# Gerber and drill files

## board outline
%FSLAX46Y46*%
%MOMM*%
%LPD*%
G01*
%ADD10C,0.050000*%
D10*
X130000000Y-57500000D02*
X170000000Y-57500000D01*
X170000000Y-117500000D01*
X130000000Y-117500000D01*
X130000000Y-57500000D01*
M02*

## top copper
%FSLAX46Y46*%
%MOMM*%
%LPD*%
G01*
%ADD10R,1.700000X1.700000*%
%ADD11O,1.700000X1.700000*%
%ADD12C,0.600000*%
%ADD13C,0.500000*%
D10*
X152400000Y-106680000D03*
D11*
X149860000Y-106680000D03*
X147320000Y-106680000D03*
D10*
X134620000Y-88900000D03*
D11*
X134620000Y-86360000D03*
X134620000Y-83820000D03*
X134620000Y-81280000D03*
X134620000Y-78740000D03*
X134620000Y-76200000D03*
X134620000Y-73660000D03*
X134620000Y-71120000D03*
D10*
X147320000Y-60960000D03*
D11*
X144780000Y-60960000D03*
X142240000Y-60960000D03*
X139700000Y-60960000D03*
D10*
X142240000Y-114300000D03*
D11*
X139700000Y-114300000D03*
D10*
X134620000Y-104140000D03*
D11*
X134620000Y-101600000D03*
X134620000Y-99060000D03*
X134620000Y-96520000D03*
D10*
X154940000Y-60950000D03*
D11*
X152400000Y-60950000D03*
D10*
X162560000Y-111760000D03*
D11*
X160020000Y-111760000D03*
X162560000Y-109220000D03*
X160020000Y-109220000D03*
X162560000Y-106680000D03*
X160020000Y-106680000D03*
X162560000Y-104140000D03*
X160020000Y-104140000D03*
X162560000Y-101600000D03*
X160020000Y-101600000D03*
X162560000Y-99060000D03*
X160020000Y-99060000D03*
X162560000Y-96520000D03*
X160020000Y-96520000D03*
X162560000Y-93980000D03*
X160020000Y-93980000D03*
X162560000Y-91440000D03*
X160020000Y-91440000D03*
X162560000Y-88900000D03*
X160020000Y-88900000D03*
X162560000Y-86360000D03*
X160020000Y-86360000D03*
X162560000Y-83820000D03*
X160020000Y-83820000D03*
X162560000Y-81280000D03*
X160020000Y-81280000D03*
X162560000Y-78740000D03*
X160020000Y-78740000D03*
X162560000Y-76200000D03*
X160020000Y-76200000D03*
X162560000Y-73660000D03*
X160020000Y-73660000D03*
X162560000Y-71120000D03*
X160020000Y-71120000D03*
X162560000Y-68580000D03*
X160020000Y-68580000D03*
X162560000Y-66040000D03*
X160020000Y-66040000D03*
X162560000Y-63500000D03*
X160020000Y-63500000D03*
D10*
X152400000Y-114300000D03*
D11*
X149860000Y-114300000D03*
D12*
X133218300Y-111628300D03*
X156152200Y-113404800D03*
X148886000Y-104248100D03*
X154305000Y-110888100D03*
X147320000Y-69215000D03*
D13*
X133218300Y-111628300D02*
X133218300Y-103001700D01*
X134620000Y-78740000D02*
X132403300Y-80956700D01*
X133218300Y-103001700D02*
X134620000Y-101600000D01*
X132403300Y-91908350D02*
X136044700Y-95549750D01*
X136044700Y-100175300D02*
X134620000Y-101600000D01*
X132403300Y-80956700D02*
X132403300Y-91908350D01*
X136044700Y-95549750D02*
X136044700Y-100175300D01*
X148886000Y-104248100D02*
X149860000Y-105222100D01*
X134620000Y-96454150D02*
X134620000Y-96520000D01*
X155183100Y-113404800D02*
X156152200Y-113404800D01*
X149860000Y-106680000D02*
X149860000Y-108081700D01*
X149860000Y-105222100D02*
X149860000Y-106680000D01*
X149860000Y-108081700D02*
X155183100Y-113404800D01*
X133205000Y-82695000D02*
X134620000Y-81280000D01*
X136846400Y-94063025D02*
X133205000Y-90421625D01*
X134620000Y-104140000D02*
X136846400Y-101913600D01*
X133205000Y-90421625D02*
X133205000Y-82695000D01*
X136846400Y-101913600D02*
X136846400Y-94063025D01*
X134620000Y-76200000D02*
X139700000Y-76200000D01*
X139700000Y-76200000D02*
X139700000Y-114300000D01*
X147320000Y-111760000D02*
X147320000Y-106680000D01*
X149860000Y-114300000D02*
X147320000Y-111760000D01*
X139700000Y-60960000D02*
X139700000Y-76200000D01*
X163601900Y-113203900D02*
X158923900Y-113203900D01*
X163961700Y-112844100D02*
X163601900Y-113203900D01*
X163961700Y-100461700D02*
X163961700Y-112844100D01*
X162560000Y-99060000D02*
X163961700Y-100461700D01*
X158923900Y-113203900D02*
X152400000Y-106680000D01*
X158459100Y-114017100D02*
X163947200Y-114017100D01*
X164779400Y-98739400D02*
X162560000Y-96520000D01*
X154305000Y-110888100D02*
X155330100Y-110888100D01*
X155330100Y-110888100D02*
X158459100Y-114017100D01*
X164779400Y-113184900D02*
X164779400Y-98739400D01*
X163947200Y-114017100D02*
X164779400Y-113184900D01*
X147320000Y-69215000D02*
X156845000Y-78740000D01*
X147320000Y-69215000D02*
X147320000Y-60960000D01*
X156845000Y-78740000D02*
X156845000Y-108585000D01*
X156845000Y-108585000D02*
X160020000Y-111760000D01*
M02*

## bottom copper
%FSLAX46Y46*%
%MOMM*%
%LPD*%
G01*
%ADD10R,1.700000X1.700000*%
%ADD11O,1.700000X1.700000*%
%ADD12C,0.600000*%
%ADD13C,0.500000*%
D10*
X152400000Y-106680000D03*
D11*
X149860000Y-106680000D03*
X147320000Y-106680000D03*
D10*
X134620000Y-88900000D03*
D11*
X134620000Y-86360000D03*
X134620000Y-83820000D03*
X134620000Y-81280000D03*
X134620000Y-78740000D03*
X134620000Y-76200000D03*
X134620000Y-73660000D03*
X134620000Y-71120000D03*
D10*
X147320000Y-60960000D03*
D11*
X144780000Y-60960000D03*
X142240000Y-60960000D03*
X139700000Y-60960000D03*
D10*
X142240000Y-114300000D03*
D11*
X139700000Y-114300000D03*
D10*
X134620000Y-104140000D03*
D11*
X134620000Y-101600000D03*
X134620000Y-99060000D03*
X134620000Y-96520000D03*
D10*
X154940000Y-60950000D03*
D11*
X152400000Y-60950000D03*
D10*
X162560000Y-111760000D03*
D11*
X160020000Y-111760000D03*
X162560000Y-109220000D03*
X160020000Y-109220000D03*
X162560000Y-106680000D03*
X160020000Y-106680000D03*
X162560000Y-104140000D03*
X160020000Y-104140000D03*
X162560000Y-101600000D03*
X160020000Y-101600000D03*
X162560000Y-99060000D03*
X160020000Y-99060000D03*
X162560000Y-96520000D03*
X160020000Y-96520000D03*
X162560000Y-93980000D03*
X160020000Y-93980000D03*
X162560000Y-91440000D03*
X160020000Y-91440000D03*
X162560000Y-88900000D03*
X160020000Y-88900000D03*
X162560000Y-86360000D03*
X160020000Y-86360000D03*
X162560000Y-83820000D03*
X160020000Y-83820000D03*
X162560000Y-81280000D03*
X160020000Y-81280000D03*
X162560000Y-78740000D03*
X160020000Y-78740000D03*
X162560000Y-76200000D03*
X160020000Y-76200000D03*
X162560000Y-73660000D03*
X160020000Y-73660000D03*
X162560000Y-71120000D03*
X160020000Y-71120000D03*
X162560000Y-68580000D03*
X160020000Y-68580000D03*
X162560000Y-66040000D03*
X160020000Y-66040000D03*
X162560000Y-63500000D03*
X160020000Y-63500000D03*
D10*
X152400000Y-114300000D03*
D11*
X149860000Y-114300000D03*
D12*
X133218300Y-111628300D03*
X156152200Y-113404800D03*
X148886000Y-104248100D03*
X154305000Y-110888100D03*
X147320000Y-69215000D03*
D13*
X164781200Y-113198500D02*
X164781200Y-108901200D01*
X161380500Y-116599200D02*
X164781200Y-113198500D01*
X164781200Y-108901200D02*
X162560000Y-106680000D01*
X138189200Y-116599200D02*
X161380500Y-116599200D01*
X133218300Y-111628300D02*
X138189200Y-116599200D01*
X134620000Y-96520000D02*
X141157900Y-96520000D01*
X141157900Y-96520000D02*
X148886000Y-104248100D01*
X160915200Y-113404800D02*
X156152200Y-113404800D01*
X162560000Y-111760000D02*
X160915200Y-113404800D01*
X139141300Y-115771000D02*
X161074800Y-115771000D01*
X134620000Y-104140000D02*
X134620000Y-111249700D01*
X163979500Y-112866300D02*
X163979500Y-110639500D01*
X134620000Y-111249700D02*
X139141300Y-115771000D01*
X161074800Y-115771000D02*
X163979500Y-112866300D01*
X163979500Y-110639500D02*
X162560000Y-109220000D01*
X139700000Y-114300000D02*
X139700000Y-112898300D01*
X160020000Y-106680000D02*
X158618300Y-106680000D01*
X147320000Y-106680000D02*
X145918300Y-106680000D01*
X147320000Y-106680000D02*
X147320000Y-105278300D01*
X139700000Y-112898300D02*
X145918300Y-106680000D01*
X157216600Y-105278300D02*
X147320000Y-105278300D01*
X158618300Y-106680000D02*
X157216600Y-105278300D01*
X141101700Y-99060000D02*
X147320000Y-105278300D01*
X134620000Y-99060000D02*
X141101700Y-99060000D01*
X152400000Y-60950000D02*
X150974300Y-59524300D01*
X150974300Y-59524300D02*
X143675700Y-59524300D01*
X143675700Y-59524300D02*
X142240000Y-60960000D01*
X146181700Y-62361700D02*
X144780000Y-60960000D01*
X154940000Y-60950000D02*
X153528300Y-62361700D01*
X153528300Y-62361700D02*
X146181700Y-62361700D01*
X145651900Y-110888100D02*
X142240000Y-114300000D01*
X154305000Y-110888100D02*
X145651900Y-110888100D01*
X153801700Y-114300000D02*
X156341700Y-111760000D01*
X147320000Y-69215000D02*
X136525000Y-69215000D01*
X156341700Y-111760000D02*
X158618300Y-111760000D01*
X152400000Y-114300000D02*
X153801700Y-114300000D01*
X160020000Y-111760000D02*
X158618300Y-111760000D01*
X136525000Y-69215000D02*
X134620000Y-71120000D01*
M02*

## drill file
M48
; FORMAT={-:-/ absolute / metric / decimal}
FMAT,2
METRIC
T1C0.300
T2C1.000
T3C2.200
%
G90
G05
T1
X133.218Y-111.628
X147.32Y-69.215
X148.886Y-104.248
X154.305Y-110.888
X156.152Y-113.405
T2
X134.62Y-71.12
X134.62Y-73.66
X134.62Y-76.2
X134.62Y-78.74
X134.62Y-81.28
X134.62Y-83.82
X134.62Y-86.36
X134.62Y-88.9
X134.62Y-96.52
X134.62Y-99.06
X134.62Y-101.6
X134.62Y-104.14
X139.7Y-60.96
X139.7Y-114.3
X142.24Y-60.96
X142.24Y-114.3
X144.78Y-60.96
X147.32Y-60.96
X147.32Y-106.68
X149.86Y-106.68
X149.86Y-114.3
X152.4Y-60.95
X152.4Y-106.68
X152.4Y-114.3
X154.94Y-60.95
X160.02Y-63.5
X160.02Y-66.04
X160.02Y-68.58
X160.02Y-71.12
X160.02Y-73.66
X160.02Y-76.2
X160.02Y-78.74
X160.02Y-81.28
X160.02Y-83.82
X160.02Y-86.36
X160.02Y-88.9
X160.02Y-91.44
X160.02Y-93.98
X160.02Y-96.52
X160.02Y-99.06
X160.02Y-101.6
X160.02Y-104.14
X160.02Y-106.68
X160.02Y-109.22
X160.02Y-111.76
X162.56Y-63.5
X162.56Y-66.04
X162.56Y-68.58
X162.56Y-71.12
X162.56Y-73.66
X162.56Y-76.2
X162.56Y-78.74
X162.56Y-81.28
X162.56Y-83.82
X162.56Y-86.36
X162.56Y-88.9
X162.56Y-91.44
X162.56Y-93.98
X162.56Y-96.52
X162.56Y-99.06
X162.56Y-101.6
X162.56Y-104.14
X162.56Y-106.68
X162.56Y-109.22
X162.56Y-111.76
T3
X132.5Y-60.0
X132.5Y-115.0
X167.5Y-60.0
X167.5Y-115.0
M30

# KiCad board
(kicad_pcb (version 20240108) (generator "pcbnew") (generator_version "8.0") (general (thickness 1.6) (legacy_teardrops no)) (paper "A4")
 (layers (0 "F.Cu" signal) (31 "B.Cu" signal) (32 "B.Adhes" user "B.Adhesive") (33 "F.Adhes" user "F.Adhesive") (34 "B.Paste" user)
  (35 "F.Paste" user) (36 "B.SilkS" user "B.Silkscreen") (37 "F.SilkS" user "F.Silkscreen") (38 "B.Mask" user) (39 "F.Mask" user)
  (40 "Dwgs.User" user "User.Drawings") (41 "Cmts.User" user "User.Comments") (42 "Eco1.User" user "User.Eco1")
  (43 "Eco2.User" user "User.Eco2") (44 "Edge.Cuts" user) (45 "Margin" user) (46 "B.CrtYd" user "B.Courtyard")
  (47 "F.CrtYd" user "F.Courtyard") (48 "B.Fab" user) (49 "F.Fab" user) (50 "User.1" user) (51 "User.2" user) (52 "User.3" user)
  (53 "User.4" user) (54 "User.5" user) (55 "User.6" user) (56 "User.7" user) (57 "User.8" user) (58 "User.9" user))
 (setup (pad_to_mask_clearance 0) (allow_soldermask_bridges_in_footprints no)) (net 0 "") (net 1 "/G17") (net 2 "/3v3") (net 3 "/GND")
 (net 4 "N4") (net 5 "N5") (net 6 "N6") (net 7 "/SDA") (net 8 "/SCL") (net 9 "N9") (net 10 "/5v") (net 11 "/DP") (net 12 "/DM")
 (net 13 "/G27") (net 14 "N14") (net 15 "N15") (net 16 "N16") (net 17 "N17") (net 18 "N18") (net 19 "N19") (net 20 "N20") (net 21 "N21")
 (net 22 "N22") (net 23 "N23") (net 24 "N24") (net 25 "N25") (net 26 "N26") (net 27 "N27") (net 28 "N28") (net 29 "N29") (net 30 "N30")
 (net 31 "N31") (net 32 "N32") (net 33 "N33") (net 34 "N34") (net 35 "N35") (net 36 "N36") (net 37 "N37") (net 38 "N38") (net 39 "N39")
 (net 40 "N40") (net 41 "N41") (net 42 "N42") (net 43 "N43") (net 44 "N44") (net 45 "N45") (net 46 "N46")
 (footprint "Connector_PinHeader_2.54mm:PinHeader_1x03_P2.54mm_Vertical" (layer "F.Cu") (at 152.4 106.68 -90)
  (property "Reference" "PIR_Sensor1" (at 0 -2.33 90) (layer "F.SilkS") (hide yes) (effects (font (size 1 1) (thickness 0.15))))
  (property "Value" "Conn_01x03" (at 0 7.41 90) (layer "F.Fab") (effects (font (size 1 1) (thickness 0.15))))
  (pad "1" thru_hole rect (at 0 0 270) (size 1.7 1.7) (drill 1) (layers "*.Cu" "*.Mask") (remove_unused_layers no) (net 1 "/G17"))
  (pad "2" thru_hole oval (at 0 2.54 270) (size 1.7 1.7) (drill 1) (layers "*.Cu" "*.Mask") (remove_unused_layers no) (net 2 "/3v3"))
  (pad "3" thru_hole oval (at 0 5.08 270) (size 1.7 1.7) (drill 1) (layers "*.Cu" "*.Mask") (remove_unused_layers no) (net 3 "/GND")))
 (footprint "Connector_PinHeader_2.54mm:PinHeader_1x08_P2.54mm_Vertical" (layer "F.Cu") (at 134.62 88.9 180)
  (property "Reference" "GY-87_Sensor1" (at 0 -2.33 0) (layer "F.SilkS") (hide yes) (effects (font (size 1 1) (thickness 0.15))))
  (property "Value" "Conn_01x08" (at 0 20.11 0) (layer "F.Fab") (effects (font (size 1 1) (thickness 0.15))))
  (pad "1" thru_hole rect (at 0 0 180) (size 1.7 1.7) (drill 1) (layers "*.Cu" "*.Mask") (remove_unused_layers no) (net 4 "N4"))
  (pad "2" thru_hole oval (at 0 2.54 180) (size 1.7 1.7) (drill 1) (layers "*.Cu" "*.Mask") (remove_unused_layers no) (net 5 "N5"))
  (pad "3" thru_hole oval (at 0 5.08 180) (size 1.7 1.7) (drill 1) (layers "*.Cu" "*.Mask") (remove_unused_layers no) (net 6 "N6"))
  (pad "4" thru_hole oval (at 0 7.62 180) (size 1.7 1.7) (drill 1) (layers "*.Cu" "*.Mask") (remove_unused_layers no) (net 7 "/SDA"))
  (pad "5" thru_hole oval (at 0 10.16 180) (size 1.7 1.7) (drill 1) (layers "*.Cu" "*.Mask") (remove_unused_layers no) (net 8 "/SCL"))
  (pad "6" thru_hole oval (at 0 12.7 180) (size 1.7 1.7) (drill 1) (layers "*.Cu" "*.Mask") (remove_unused_layers no) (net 3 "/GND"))
  (pad "7" thru_hole oval (at 0 15.24 180) (size 1.7 1.7) (drill 1) (layers "*.Cu" "*.Mask") (remove_unused_layers no) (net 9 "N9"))
  (pad "8" thru_hole oval (at 0 17.78 180) (size 1.7 1.7) (drill 1) (layers "*.Cu" "*.Mask") (remove_unused_layers no) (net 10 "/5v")))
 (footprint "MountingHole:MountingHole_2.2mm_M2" (layer "F.Cu") (at 132.5 60)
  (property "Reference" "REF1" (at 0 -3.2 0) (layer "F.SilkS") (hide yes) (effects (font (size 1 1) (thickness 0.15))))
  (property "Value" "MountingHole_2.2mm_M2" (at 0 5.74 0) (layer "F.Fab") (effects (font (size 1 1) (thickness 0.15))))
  (pad "" np_thru_hole circle (at 0 0) (size 2.2 2.2) (drill 2.2) (layers "*.Cu" "*.Mask")))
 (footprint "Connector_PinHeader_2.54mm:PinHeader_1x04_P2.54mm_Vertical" (layer "F.Cu") (at 147.32 60.96 -90)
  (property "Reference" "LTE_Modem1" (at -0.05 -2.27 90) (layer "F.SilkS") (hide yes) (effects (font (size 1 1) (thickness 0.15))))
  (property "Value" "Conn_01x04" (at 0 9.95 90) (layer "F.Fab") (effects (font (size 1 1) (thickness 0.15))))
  (pad "1" thru_hole rect (at 0 0 270) (size 1.7 1.7) (drill 1) (layers "*.Cu" "*.Mask") (remove_unused_layers no) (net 10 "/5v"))
  (pad "2" thru_hole oval (at 0 2.54 270) (size 1.7 1.7) (drill 1) (layers "*.Cu" "*.Mask") (remove_unused_layers no) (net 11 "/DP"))
  (pad "3" thru_hole oval (at 0 5.08 270) (size 1.7 1.7) (drill 1) (layers "*.Cu" "*.Mask") (remove_unused_layers no) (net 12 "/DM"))
  (pad "4" thru_hole oval (at 0 7.62 270) (size 1.7 1.7) (drill 1) (layers "*.Cu" "*.Mask") (remove_unused_layers no) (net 3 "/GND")))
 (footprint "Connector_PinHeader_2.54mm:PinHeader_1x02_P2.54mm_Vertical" (layer "F.Cu") (at 142.24 114.3 -90)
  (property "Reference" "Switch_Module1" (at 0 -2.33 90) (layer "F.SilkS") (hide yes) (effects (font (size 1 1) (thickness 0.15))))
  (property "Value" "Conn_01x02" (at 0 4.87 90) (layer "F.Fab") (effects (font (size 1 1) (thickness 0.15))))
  (pad "1" thru_hole rect (at 0 0 270) (size 1.7 1.7) (drill 1) (layers "*.Cu" "*.Mask") (remove_unused_layers no) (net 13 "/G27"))
  (pad "2" thru_hole oval (at 0 2.54 270) (size 1.7 1.7) (drill 1) (layers "*.Cu" "*.Mask") (remove_unused_layers no) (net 3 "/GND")))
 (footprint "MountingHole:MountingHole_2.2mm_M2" (layer "F.Cu") (at 167.5 115)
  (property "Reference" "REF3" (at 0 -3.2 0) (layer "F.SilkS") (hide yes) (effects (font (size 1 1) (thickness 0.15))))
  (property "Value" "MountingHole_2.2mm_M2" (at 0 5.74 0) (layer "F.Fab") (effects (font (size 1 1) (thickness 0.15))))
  (pad "" np_thru_hole circle (at 0 0) (size 2.2 2.2) (drill 2.2) (layers "*.Cu" "*.Mask")))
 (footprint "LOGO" (layer "F.Cu") (at 144.78 97.79)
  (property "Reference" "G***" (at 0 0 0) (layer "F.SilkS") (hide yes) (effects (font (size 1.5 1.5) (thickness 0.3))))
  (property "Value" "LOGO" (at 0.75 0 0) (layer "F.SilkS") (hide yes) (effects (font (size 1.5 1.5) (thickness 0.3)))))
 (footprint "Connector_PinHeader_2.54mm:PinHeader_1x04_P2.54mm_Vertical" (layer "F.Cu") (at 134.62 104.14 180)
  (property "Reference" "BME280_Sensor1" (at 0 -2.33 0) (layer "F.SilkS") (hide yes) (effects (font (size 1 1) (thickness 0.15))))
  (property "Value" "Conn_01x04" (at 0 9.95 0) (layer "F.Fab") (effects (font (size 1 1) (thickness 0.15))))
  (pad "1" thru_hole rect (at 0 0 180) (size 1.7 1.7) (drill 1) (layers "*.Cu" "*.Mask") (remove_unused_layers no) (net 7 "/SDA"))
  (pad "2" thru_hole oval (at 0 2.54 180) (size 1.7 1.7) (drill 1) (layers "*.Cu" "*.Mask") (remove_unused_layers no) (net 8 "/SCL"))
  (pad "3" thru_hole oval (at 0 5.08 180) (size 1.7 1.7) (drill 1) (layers "*.Cu" "*.Mask") (remove_unused_layers no) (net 3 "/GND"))
  (pad "4" thru_hole oval (at 0 7.62 180) (size 1.7 1.7) (drill 1) (layers "*.Cu" "*.Mask") (remove_unused_layers no) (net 2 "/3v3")))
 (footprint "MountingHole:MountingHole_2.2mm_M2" (layer "F.Cu") (at 132.5 115)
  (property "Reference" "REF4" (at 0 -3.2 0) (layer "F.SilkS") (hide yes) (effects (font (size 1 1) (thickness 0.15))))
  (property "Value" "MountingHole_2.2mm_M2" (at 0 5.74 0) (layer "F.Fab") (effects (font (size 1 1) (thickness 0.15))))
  (pad "" np_thru_hole circle (at 0 0) (size 2.2 2.2) (drill 2.2) (layers "*.Cu" "*.Mask")))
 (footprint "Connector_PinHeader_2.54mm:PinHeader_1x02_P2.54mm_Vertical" (layer "F.Cu") (at 154.94 60.95 -90)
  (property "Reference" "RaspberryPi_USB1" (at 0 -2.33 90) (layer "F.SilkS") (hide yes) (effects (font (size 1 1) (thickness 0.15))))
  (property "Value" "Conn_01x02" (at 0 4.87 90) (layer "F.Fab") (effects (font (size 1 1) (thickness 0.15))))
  (pad "1" thru_hole rect (at 0 0 270) (size 1.7 1.7) (drill 1) (layers "*.Cu" "*.Mask") (remove_unused_layers no) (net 11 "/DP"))
  (pad "2" thru_hole oval (at 0 2.54 270) (size 1.7 1.7) (drill 1) (layers "*.Cu" "*.Mask") (remove_unused_layers no) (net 12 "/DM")))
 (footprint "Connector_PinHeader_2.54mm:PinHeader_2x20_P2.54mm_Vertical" (layer "F.Cu") (at 162.56 111.76 180)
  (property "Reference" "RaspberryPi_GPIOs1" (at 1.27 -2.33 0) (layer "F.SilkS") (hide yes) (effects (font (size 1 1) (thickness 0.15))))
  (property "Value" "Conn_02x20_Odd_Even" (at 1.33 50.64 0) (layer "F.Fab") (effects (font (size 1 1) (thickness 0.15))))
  (pad "1" thru_hole rect (at 0 0 180) (size 1.7 1.7) (drill 1) (layers "*.Cu" "*.Mask") (remove_unused_layers no) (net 2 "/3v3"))
  (pad "2" thru_hole oval (at 2.54 0 180) (size 1.7 1.7) (drill 1) (layers "*.Cu" "*.Mask") (remove_unused_layers no) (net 10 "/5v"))
  (pad "3" thru_hole oval (at 0 2.54 180) (size 1.7 1.7) (drill 1) (layers "*.Cu" "*.Mask") (remove_unused_layers no) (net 7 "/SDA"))
  (pad "4" thru_hole oval (at 2.54 2.54 180) (size 1.7 1.7) (drill 1) (layers "*.Cu" "*.Mask") (remove_unused_layers no) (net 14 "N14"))
  (pad "5" thru_hole oval (at 0 5.08 180) (size 1.7 1.7) (drill 1) (layers "*.Cu" "*.Mask") (remove_unused_layers no) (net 8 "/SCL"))
  (pad "6" thru_hole oval (at 2.54 5.08 180) (size 1.7 1.7) (drill 1) (layers "*.Cu" "*.Mask") (remove_unused_layers no) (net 3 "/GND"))
  (pad "7" thru_hole oval (at 0 7.62 180) (size 1.7 1.7) (drill 1) (layers "*.Cu" "*.Mask") (remove_unused_layers no) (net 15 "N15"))
  (pad "8" thru_hole oval (at 2.54 7.62 180) (size 1.7 1.7) (drill 1) (layers "*.Cu" "*.Mask") (remove_unused_layers no) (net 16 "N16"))
  (pad "9" thru_hole oval (at 0 10.16 180) (size 1.7 1.7) (drill 1) (layers "*.Cu" "*.Mask") (remove_unused_layers no) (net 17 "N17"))
  (pad "10" thru_hole oval (at 2.54 10.16 180) (size 1.7 1.7) (drill 1) (layers "*.Cu" "*.Mask") (remove_unused_layers no) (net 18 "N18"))
  (pad "11" thru_hole oval (at 0 12.7 180) (size 1.7 1.7) (drill 1) (layers "*.Cu" "*.Mask") (remove_unused_layers no) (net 1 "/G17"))
  (pad "12" thru_hole oval (at 2.54 12.7 180) (size 1.7 1.7) (drill 1) (layers "*.Cu" "*.Mask") (remove_unused_layers no) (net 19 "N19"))
  (pad "13" thru_hole oval (at 0 15.24 180) (size 1.7 1.7) (drill 1) (layers "*.Cu" "*.Mask") (remove_unused_layers no) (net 13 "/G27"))
  (pad "14" thru_hole oval (at 2.54 15.24 180) (size 1.7 1.7) (drill 1) (layers "*.Cu" "*.Mask") (remove_unused_layers no) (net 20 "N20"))
  (pad "15" thru_hole oval (at 0 17.78 180) (size 1.7 1.7) (drill 1) (layers "*.Cu" "*.Mask") (remove_unused_layers no) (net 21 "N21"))
  (pad "16" thru_hole oval (at 2.54 17.78 180) (size 1.7 1.7) (drill 1) (layers "*.Cu" "*.Mask") (remove_unused_layers no) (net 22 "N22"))
  (pad "17" thru_hole oval (at 0 20.32 180) (size 1.7 1.7) (drill 1) (layers "*.Cu" "*.Mask") (remove_unused_layers no) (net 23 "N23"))
  (pad "18" thru_hole oval (at 2.54 20.32 180) (size 1.7 1.7) (drill 1) (layers "*.Cu" "*.Mask") (remove_unused_layers no) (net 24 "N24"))
  (pad "19" thru_hole oval (at 0 22.86 180) (size 1.7 1.7) (drill 1) (layers "*.Cu" "*.Mask") (remove_unused_layers no) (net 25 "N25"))
  (pad "20" thru_hole oval (at 2.54 22.86 180) (size 1.7 1.7) (drill 1) (layers "*.Cu" "*.Mask") (remove_unused_layers no) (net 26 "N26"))
  (pad "21" thru_hole oval (at 0 25.4 180) (size 1.7 1.7) (drill 1) (layers "*.Cu" "*.Mask") (remove_unused_layers no) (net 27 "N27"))
  (pad "22" thru_hole oval (at 2.54 25.4 180) (size 1.7 1.7) (drill 1) (layers "*.Cu" "*.Mask") (remove_unused_layers no) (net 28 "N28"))
  (pad "23" thru_hole oval (at 0 27.94 180) (size 1.7 1.7) (drill 1) (layers "*.Cu" "*.Mask") (remove_unused_layers no) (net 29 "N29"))
  (pad "24" thru_hole oval (at 2.54 27.94 180) (size 1.7 1.7) (drill 1) (layers "*.Cu" "*.Mask") (remove_unused_layers no) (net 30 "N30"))
  (pad "25" thru_hole oval (at 0 30.48 180) (size 1.7 1.7) (drill 1) (layers "*.Cu" "*.Mask") (remove_unused_layers no) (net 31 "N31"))
  (pad "26" thru_hole oval (at 2.54 30.48 180) (size 1.7 1.7) (drill 1) (layers "*.Cu" "*.Mask") (remove_unused_layers no) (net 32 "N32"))
  (pad "27" thru_hole oval (at 0 33.02 180) (size 1.7 1.7) (drill 1) (layers "*.Cu" "*.Mask") (remove_unused_layers no) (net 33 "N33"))
  (pad "28" thru_hole oval (at 2.54 33.02 180) (size 1.7 1.7) (drill 1) (layers "*.Cu" "*.Mask") (remove_unused_layers no) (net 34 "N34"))
  (pad "29" thru_hole oval (at 0 35.56 180) (size 1.7 1.7) (drill 1) (layers "*.Cu" "*.Mask") (remove_unused_layers no) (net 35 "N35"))
  (pad "30" thru_hole oval (at 2.54 35.56 180) (size 1.7 1.7) (drill 1) (layers "*.Cu" "*.Mask") (remove_unused_layers no) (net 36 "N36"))
  (pad "31" thru_hole oval (at 0 38.1 180) (size 1.7 1.7) (drill 1) (layers "*.Cu" "*.Mask") (remove_unused_layers no) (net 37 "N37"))
  (pad "32" thru_hole oval (at 2.54 38.1 180) (size 1.7 1.7) (drill 1) (layers "*.Cu" "*.Mask") (remove_unused_layers no) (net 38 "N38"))
  (pad "33" thru_hole oval (at 0 40.64 180) (size 1.7 1.7) (drill 1) (layers "*.Cu" "*.Mask") (remove_unused_layers no) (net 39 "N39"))
  (pad "34" thru_hole oval (at 2.54 40.64 180) (size 1.7 1.7) (drill 1) (layers "*.Cu" "*.Mask") (remove_unused_layers no) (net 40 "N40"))
  (pad "35" thru_hole oval (at 0 43.18 180) (size 1.7 1.7) (drill 1) (layers "*.Cu" "*.Mask") (remove_unused_layers no) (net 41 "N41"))
  (pad "36" thru_hole oval (at 2.54 43.18 180) (size 1.7 1.7) (drill 1) (layers "*.Cu" "*.Mask") (remove_unused_layers no) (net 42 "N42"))
  (pad "37" thru_hole oval (at 0 45.72 180) (size 1.7 1.7) (drill 1) (layers "*.Cu" "*.Mask") (remove_unused_layers no) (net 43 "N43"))
  (pad "38" thru_hole oval (at 2.54 45.72 180) (size 1.7 1.7) (drill 1) (layers "*.Cu" "*.Mask") (remove_unused_layers no) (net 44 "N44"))
  (pad "39" thru_hole oval (at 0 48.26 180) (size 1.7 1.7) (drill 1) (layers "*.Cu" "*.Mask") (remove_unused_layers no) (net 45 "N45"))
  (pad "40" thru_hole oval (at 2.54 48.26 180) (size 1.7 1.7) (drill 1) (layers "*.Cu" "*.Mask") (remove_unused_layers no) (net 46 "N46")))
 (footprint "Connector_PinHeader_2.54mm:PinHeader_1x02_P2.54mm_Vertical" (layer "F.Cu") (at 152.4 114.3 -90)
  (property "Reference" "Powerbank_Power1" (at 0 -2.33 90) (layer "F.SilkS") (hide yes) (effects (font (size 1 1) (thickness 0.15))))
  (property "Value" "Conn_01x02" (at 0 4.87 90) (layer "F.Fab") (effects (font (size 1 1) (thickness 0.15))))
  (pad "1" thru_hole rect (at 0 0 270) (size 1.7 1.7) (drill 1) (layers "*.Cu" "*.Mask") (remove_unused_layers no) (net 10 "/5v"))
  (pad "2" thru_hole oval (at 0 2.54 270) (size 1.7 1.7) (drill 1) (layers "*.Cu" "*.Mask") (remove_unused_layers no) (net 3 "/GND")))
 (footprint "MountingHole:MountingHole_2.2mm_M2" (layer "F.Cu") (at 167.5 60)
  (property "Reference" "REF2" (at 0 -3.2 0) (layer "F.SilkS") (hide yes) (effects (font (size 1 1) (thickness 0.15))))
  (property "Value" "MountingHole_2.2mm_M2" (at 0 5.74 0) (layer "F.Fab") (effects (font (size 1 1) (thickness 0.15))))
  (pad "" np_thru_hole circle (at 0 0) (size 2.2 2.2) (drill 2.2) (layers "*.Cu" "*.Mask")))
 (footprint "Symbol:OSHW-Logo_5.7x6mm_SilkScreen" (layer "F.Cu") (at 152.4 97.79)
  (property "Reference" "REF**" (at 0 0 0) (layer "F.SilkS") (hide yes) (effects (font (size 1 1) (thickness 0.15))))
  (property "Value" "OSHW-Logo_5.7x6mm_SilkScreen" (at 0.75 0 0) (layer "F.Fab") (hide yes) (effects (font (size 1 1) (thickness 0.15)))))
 (gr_rect (start 130 57.5) (end 170 117.5) (stroke (width 0.05) (type default)) (fill none) (layer "Edge.Cuts"))
 (segment (start 133.2183 111.6283) (end 133.2183 103.0017) (width 0.5) (layer "F.Cu") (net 8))
 (segment (start 134.62 78.74) (end 132.4033 80.9567) (width 0.5) (layer "F.Cu") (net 8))
 (segment (start 133.2183 103.0017) (end 134.62 101.6) (width 0.5) (layer "F.Cu") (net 8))
 (segment (start 132.4033 91.90835) (end 136.0447 95.54975) (width 0.5) (layer "F.Cu") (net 8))
 (segment (start 136.0447 100.1753) (end 134.62 101.6) (width 0.5) (layer "F.Cu") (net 8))
 (segment (start 132.4033 80.9567) (end 132.4033 91.90835) (width 0.5) (layer "F.Cu") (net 8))
 (segment (start 136.0447 95.54975) (end 136.0447 100.1753) (width 0.5) (layer "F.Cu") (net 8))
 (via (at 133.2183 111.6283) (size 0.6) (drill 0.3) (layers "F.Cu" "B.Cu") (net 8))
 (segment (start 164.7812 113.1985) (end 164.7812 108.9012) (width 0.5) (layer "B.Cu") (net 8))
 (segment (start 161.3805 116.5992) (end 164.7812 113.1985) (width 0.5) (layer "B.Cu") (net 8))
 (segment (start 164.7812 108.9012) (end 162.56 106.68) (width 0.5) (layer "B.Cu") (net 8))
 (segment (start 138.1892 116.5992) (end 161.3805 116.5992) (width 0.5) (layer "B.Cu") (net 8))
 (segment (start 133.2183 111.6283) (end 138.1892 116.5992) (width 0.5) (layer "B.Cu") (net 8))
 (segment (start 148.886 104.2481) (end 149.86 105.2221) (width 0.5) (layer "F.Cu") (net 2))
 (segment (start 134.62 96.45415) (end 134.62 96.52) (width 0.5) (layer "F.Cu") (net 2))
 (segment (start 155.1831 113.4048) (end 156.1522 113.4048) (width 0.5) (layer "F.Cu") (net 2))
 (segment (start 149.86 106.68) (end 149.86 108.0817) (width 0.5) (layer "F.Cu") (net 2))
 (segment (start 149.86 105.2221) (end 149.86 106.68) (width 0.5) (layer "F.Cu") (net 2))
 (segment (start 149.86 108.0817) (end 155.1831 113.4048) (width 0.5) (layer "F.Cu") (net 2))
 (via (at 156.1522 113.4048) (size 0.6) (drill 0.3) (layers "F.Cu" "B.Cu") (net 2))
 (via (at 148.886 104.2481) (size 0.6) (drill 0.3) (layers "F.Cu" "B.Cu") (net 2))
 (segment (start 134.62 96.52) (end 141.1579 96.52) (width 0.5) (layer "B.Cu") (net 2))
 (segment (start 141.1579 96.52) (end 148.886 104.2481) (width 0.5) (layer "B.Cu") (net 2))
 (segment (start 160.9152 113.4048) (end 156.1522 113.4048) (width 0.5) (layer "B.Cu") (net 2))
 (segment (start 162.56 111.76) (end 160.9152 113.4048) (width 0.5) (layer "B.Cu") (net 2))
 (segment (start 133.205 82.695) (end 134.62 81.28) (width 0.5) (layer "F.Cu") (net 7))
 (segment (start 136.8464 94.063025) (end 133.205 90.421625) (width 0.5) (layer "F.Cu") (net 7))
 (segment (start 134.62 104.14) (end 136.8464 101.9136) (width 0.5) (layer "F.Cu") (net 7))
 (segment (start 133.205 90.421625) (end 133.205 82.695) (width 0.5) (layer "F.Cu") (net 7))
 (segment (start 136.8464 101.9136) (end 136.8464 94.063025) (width 0.5) (layer "F.Cu") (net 7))
 (segment (start 139.1413 115.771) (end 161.0748 115.771) (width 0.5) (layer "B.Cu") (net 7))
 (segment (start 134.62 104.14) (end 134.62 111.2497) (width 0.5) (layer "B.Cu") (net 7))
 (segment (start 163.9795 112.8663) (end 163.9795 110.6395) (width 0.5) (layer "B.Cu") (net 7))
 (segment (start 134.62 111.2497) (end 139.1413 115.771) (width 0.5) (layer "B.Cu") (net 7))
 (segment (start 161.0748 115.771) (end 163.9795 112.8663) (width 0.5) (layer "B.Cu") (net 7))
 (segment (start 163.9795 110.6395) (end 162.56 109.22) (width 0.5) (layer "B.Cu") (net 7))
 (segment (start 134.62 76.2) (end 139.7 76.2) (width 0.5) (layer "F.Cu") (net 3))
 (segment (start 139.7 76.2) (end 139.7 114.3) (width 0.5) (layer "F.Cu") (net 3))
 (segment (start 147.32 111.76) (end 147.32 106.68) (width 0.5) (layer "F.Cu") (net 3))
 (segment (start 149.86 114.3) (end 147.32 111.76) (width 0.5) (layer "F.Cu") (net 3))
 (segment (start 139.7 60.96) (end 139.7 76.2) (width 0.5) (layer "F.Cu") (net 3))
 (segment (start 139.7 114.3) (end 139.7 112.8983) (width 0.5) (layer "B.Cu") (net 3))
 (segment (start 160.02 106.68) (end 158.6183 106.68) (width 0.5) (layer "B.Cu") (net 3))
 (segment (start 147.32 106.68) (end 145.9183 106.68) (width 0.5) (layer "B.Cu") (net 3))
 (segment (start 147.32 106.68) (end 147.32 105.2783) (width 0.5) (layer "B.Cu") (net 3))
 (segment (start 139.7 112.8983) (end 145.9183 106.68) (width 0.5) (layer "B.Cu") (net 3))
 (segment (start 157.2166 105.2783) (end 147.32 105.2783) (width 0.5) (layer "B.Cu") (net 3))
 (segment (start 158.6183 106.68) (end 157.2166 105.2783) (width 0.5) (layer "B.Cu") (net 3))
 (segment (start 141.1017 99.06) (end 147.32 105.2783) (width 0.5) (layer "B.Cu") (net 3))
 (segment (start 134.62 99.06) (end 141.1017 99.06) (width 0.5) (layer "B.Cu") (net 3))
 (segment (start 152.4 60.95) (end 150.9743 59.5243) (width 0.5) (layer "B.Cu") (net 12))
 (segment (start 150.9743 59.5243) (end 143.6757 59.5243) (width 0.5) (layer "B.Cu") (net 12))
 (segment (start 143.6757 59.5243) (end 142.24 60.96) (width 0.5) (layer "B.Cu") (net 12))
 (segment (start 146.1817 62.3617) (end 144.78 60.96) (width 0.5) (layer "B.Cu") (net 11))
 (segment (start 154.94 60.95) (end 153.5283 62.3617) (width 0.5) (layer "B.Cu") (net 11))
 (segment (start 153.5283 62.3617) (end 146.1817 62.3617) (width 0.5) (layer "B.Cu") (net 11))
 (segment (start 163.6019 113.2039) (end 158.9239 113.2039) (width 0.5) (layer "F.Cu") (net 1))
 (segment (start 163.9617 112.8441) (end 163.6019 113.2039) (width 0.5) (layer "F.Cu") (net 1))
 (segment (start 163.9617 100.4617) (end 163.9617 112.8441) (width 0.5) (layer "F.Cu") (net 1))
 (segment (start 162.56 99.06) (end 163.9617 100.4617) (width 0.5) (layer "F.Cu") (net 1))
 (segment (start 158.9239 113.2039) (end 152.4 106.68) (width 0.5) (layer "F.Cu") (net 1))
 (segment (start 158.4591 114.0171) (end 163.9472 114.0171) (width 0.5) (layer "F.Cu") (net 13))
 (segment (start 164.7794 98.7394) (end 162.56 96.52) (width 0.5) (layer "F.Cu") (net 13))
 (segment (start 154.305 110.8881) (end 155.3301 110.8881) (width 0.5) (layer "F.Cu") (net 13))
 (segment (start 155.3301 110.8881) (end 158.4591 114.0171) (width 0.5) (layer "F.Cu") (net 13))
 (segment (start 164.7794 113.1849) (end 164.7794 98.7394) (width 0.5) (layer "F.Cu") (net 13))
 (segment (start 163.9472 114.0171) (end 164.7794 113.1849) (width 0.5) (layer "F.Cu") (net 13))
 (via (at 154.305 110.8881) (size 0.6) (drill 0.3) (layers "F.Cu" "B.Cu") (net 13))
 (segment (start 145.6519 110.8881) (end 142.24 114.3) (width 0.5) (layer "B.Cu") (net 13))
 (segment (start 154.305 110.8881) (end 145.6519 110.8881) (width 0.5) (layer "B.Cu") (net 13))
 (segment (start 147.32 69.215) (end 156.845 78.74) (width 0.5) (layer "F.Cu") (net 10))
 (segment (start 147.32 69.215) (end 147.32 60.96) (width 0.5) (layer "F.Cu") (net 10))
 (segment (start 156.845 78.74) (end 156.845 108.585) (width 0.5) (layer "F.Cu") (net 10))
 (segment (start 156.845 108.585) (end 160.02 111.76) (width 0.5) (layer "F.Cu") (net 10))
 (via (at 147.32 69.215) (size 0.6) (drill 0.3) (layers "F.Cu" "B.Cu") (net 10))
 (segment (start 153.8017 114.3) (end 156.3417 111.76) (width 0.5) (layer "B.Cu") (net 10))
 (segment (start 147.32 69.215) (end 136.525 69.215) (width 0.5) (layer "B.Cu") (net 10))
 (segment (start 156.3417 111.76) (end 158.6183 111.76) (width 0.5) (layer "B.Cu") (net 10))
 (segment (start 152.4 114.3) (end 153.8017 114.3) (width 0.5) (layer "B.Cu") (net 10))
 (segment (start 160.02 111.76) (end 158.6183 111.76) (width 0.5) (layer "B.Cu") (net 10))
 (segment (start 136.525 69.215) (end 134.62 71.12) (width 0.5) (layer "B.Cu") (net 10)))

